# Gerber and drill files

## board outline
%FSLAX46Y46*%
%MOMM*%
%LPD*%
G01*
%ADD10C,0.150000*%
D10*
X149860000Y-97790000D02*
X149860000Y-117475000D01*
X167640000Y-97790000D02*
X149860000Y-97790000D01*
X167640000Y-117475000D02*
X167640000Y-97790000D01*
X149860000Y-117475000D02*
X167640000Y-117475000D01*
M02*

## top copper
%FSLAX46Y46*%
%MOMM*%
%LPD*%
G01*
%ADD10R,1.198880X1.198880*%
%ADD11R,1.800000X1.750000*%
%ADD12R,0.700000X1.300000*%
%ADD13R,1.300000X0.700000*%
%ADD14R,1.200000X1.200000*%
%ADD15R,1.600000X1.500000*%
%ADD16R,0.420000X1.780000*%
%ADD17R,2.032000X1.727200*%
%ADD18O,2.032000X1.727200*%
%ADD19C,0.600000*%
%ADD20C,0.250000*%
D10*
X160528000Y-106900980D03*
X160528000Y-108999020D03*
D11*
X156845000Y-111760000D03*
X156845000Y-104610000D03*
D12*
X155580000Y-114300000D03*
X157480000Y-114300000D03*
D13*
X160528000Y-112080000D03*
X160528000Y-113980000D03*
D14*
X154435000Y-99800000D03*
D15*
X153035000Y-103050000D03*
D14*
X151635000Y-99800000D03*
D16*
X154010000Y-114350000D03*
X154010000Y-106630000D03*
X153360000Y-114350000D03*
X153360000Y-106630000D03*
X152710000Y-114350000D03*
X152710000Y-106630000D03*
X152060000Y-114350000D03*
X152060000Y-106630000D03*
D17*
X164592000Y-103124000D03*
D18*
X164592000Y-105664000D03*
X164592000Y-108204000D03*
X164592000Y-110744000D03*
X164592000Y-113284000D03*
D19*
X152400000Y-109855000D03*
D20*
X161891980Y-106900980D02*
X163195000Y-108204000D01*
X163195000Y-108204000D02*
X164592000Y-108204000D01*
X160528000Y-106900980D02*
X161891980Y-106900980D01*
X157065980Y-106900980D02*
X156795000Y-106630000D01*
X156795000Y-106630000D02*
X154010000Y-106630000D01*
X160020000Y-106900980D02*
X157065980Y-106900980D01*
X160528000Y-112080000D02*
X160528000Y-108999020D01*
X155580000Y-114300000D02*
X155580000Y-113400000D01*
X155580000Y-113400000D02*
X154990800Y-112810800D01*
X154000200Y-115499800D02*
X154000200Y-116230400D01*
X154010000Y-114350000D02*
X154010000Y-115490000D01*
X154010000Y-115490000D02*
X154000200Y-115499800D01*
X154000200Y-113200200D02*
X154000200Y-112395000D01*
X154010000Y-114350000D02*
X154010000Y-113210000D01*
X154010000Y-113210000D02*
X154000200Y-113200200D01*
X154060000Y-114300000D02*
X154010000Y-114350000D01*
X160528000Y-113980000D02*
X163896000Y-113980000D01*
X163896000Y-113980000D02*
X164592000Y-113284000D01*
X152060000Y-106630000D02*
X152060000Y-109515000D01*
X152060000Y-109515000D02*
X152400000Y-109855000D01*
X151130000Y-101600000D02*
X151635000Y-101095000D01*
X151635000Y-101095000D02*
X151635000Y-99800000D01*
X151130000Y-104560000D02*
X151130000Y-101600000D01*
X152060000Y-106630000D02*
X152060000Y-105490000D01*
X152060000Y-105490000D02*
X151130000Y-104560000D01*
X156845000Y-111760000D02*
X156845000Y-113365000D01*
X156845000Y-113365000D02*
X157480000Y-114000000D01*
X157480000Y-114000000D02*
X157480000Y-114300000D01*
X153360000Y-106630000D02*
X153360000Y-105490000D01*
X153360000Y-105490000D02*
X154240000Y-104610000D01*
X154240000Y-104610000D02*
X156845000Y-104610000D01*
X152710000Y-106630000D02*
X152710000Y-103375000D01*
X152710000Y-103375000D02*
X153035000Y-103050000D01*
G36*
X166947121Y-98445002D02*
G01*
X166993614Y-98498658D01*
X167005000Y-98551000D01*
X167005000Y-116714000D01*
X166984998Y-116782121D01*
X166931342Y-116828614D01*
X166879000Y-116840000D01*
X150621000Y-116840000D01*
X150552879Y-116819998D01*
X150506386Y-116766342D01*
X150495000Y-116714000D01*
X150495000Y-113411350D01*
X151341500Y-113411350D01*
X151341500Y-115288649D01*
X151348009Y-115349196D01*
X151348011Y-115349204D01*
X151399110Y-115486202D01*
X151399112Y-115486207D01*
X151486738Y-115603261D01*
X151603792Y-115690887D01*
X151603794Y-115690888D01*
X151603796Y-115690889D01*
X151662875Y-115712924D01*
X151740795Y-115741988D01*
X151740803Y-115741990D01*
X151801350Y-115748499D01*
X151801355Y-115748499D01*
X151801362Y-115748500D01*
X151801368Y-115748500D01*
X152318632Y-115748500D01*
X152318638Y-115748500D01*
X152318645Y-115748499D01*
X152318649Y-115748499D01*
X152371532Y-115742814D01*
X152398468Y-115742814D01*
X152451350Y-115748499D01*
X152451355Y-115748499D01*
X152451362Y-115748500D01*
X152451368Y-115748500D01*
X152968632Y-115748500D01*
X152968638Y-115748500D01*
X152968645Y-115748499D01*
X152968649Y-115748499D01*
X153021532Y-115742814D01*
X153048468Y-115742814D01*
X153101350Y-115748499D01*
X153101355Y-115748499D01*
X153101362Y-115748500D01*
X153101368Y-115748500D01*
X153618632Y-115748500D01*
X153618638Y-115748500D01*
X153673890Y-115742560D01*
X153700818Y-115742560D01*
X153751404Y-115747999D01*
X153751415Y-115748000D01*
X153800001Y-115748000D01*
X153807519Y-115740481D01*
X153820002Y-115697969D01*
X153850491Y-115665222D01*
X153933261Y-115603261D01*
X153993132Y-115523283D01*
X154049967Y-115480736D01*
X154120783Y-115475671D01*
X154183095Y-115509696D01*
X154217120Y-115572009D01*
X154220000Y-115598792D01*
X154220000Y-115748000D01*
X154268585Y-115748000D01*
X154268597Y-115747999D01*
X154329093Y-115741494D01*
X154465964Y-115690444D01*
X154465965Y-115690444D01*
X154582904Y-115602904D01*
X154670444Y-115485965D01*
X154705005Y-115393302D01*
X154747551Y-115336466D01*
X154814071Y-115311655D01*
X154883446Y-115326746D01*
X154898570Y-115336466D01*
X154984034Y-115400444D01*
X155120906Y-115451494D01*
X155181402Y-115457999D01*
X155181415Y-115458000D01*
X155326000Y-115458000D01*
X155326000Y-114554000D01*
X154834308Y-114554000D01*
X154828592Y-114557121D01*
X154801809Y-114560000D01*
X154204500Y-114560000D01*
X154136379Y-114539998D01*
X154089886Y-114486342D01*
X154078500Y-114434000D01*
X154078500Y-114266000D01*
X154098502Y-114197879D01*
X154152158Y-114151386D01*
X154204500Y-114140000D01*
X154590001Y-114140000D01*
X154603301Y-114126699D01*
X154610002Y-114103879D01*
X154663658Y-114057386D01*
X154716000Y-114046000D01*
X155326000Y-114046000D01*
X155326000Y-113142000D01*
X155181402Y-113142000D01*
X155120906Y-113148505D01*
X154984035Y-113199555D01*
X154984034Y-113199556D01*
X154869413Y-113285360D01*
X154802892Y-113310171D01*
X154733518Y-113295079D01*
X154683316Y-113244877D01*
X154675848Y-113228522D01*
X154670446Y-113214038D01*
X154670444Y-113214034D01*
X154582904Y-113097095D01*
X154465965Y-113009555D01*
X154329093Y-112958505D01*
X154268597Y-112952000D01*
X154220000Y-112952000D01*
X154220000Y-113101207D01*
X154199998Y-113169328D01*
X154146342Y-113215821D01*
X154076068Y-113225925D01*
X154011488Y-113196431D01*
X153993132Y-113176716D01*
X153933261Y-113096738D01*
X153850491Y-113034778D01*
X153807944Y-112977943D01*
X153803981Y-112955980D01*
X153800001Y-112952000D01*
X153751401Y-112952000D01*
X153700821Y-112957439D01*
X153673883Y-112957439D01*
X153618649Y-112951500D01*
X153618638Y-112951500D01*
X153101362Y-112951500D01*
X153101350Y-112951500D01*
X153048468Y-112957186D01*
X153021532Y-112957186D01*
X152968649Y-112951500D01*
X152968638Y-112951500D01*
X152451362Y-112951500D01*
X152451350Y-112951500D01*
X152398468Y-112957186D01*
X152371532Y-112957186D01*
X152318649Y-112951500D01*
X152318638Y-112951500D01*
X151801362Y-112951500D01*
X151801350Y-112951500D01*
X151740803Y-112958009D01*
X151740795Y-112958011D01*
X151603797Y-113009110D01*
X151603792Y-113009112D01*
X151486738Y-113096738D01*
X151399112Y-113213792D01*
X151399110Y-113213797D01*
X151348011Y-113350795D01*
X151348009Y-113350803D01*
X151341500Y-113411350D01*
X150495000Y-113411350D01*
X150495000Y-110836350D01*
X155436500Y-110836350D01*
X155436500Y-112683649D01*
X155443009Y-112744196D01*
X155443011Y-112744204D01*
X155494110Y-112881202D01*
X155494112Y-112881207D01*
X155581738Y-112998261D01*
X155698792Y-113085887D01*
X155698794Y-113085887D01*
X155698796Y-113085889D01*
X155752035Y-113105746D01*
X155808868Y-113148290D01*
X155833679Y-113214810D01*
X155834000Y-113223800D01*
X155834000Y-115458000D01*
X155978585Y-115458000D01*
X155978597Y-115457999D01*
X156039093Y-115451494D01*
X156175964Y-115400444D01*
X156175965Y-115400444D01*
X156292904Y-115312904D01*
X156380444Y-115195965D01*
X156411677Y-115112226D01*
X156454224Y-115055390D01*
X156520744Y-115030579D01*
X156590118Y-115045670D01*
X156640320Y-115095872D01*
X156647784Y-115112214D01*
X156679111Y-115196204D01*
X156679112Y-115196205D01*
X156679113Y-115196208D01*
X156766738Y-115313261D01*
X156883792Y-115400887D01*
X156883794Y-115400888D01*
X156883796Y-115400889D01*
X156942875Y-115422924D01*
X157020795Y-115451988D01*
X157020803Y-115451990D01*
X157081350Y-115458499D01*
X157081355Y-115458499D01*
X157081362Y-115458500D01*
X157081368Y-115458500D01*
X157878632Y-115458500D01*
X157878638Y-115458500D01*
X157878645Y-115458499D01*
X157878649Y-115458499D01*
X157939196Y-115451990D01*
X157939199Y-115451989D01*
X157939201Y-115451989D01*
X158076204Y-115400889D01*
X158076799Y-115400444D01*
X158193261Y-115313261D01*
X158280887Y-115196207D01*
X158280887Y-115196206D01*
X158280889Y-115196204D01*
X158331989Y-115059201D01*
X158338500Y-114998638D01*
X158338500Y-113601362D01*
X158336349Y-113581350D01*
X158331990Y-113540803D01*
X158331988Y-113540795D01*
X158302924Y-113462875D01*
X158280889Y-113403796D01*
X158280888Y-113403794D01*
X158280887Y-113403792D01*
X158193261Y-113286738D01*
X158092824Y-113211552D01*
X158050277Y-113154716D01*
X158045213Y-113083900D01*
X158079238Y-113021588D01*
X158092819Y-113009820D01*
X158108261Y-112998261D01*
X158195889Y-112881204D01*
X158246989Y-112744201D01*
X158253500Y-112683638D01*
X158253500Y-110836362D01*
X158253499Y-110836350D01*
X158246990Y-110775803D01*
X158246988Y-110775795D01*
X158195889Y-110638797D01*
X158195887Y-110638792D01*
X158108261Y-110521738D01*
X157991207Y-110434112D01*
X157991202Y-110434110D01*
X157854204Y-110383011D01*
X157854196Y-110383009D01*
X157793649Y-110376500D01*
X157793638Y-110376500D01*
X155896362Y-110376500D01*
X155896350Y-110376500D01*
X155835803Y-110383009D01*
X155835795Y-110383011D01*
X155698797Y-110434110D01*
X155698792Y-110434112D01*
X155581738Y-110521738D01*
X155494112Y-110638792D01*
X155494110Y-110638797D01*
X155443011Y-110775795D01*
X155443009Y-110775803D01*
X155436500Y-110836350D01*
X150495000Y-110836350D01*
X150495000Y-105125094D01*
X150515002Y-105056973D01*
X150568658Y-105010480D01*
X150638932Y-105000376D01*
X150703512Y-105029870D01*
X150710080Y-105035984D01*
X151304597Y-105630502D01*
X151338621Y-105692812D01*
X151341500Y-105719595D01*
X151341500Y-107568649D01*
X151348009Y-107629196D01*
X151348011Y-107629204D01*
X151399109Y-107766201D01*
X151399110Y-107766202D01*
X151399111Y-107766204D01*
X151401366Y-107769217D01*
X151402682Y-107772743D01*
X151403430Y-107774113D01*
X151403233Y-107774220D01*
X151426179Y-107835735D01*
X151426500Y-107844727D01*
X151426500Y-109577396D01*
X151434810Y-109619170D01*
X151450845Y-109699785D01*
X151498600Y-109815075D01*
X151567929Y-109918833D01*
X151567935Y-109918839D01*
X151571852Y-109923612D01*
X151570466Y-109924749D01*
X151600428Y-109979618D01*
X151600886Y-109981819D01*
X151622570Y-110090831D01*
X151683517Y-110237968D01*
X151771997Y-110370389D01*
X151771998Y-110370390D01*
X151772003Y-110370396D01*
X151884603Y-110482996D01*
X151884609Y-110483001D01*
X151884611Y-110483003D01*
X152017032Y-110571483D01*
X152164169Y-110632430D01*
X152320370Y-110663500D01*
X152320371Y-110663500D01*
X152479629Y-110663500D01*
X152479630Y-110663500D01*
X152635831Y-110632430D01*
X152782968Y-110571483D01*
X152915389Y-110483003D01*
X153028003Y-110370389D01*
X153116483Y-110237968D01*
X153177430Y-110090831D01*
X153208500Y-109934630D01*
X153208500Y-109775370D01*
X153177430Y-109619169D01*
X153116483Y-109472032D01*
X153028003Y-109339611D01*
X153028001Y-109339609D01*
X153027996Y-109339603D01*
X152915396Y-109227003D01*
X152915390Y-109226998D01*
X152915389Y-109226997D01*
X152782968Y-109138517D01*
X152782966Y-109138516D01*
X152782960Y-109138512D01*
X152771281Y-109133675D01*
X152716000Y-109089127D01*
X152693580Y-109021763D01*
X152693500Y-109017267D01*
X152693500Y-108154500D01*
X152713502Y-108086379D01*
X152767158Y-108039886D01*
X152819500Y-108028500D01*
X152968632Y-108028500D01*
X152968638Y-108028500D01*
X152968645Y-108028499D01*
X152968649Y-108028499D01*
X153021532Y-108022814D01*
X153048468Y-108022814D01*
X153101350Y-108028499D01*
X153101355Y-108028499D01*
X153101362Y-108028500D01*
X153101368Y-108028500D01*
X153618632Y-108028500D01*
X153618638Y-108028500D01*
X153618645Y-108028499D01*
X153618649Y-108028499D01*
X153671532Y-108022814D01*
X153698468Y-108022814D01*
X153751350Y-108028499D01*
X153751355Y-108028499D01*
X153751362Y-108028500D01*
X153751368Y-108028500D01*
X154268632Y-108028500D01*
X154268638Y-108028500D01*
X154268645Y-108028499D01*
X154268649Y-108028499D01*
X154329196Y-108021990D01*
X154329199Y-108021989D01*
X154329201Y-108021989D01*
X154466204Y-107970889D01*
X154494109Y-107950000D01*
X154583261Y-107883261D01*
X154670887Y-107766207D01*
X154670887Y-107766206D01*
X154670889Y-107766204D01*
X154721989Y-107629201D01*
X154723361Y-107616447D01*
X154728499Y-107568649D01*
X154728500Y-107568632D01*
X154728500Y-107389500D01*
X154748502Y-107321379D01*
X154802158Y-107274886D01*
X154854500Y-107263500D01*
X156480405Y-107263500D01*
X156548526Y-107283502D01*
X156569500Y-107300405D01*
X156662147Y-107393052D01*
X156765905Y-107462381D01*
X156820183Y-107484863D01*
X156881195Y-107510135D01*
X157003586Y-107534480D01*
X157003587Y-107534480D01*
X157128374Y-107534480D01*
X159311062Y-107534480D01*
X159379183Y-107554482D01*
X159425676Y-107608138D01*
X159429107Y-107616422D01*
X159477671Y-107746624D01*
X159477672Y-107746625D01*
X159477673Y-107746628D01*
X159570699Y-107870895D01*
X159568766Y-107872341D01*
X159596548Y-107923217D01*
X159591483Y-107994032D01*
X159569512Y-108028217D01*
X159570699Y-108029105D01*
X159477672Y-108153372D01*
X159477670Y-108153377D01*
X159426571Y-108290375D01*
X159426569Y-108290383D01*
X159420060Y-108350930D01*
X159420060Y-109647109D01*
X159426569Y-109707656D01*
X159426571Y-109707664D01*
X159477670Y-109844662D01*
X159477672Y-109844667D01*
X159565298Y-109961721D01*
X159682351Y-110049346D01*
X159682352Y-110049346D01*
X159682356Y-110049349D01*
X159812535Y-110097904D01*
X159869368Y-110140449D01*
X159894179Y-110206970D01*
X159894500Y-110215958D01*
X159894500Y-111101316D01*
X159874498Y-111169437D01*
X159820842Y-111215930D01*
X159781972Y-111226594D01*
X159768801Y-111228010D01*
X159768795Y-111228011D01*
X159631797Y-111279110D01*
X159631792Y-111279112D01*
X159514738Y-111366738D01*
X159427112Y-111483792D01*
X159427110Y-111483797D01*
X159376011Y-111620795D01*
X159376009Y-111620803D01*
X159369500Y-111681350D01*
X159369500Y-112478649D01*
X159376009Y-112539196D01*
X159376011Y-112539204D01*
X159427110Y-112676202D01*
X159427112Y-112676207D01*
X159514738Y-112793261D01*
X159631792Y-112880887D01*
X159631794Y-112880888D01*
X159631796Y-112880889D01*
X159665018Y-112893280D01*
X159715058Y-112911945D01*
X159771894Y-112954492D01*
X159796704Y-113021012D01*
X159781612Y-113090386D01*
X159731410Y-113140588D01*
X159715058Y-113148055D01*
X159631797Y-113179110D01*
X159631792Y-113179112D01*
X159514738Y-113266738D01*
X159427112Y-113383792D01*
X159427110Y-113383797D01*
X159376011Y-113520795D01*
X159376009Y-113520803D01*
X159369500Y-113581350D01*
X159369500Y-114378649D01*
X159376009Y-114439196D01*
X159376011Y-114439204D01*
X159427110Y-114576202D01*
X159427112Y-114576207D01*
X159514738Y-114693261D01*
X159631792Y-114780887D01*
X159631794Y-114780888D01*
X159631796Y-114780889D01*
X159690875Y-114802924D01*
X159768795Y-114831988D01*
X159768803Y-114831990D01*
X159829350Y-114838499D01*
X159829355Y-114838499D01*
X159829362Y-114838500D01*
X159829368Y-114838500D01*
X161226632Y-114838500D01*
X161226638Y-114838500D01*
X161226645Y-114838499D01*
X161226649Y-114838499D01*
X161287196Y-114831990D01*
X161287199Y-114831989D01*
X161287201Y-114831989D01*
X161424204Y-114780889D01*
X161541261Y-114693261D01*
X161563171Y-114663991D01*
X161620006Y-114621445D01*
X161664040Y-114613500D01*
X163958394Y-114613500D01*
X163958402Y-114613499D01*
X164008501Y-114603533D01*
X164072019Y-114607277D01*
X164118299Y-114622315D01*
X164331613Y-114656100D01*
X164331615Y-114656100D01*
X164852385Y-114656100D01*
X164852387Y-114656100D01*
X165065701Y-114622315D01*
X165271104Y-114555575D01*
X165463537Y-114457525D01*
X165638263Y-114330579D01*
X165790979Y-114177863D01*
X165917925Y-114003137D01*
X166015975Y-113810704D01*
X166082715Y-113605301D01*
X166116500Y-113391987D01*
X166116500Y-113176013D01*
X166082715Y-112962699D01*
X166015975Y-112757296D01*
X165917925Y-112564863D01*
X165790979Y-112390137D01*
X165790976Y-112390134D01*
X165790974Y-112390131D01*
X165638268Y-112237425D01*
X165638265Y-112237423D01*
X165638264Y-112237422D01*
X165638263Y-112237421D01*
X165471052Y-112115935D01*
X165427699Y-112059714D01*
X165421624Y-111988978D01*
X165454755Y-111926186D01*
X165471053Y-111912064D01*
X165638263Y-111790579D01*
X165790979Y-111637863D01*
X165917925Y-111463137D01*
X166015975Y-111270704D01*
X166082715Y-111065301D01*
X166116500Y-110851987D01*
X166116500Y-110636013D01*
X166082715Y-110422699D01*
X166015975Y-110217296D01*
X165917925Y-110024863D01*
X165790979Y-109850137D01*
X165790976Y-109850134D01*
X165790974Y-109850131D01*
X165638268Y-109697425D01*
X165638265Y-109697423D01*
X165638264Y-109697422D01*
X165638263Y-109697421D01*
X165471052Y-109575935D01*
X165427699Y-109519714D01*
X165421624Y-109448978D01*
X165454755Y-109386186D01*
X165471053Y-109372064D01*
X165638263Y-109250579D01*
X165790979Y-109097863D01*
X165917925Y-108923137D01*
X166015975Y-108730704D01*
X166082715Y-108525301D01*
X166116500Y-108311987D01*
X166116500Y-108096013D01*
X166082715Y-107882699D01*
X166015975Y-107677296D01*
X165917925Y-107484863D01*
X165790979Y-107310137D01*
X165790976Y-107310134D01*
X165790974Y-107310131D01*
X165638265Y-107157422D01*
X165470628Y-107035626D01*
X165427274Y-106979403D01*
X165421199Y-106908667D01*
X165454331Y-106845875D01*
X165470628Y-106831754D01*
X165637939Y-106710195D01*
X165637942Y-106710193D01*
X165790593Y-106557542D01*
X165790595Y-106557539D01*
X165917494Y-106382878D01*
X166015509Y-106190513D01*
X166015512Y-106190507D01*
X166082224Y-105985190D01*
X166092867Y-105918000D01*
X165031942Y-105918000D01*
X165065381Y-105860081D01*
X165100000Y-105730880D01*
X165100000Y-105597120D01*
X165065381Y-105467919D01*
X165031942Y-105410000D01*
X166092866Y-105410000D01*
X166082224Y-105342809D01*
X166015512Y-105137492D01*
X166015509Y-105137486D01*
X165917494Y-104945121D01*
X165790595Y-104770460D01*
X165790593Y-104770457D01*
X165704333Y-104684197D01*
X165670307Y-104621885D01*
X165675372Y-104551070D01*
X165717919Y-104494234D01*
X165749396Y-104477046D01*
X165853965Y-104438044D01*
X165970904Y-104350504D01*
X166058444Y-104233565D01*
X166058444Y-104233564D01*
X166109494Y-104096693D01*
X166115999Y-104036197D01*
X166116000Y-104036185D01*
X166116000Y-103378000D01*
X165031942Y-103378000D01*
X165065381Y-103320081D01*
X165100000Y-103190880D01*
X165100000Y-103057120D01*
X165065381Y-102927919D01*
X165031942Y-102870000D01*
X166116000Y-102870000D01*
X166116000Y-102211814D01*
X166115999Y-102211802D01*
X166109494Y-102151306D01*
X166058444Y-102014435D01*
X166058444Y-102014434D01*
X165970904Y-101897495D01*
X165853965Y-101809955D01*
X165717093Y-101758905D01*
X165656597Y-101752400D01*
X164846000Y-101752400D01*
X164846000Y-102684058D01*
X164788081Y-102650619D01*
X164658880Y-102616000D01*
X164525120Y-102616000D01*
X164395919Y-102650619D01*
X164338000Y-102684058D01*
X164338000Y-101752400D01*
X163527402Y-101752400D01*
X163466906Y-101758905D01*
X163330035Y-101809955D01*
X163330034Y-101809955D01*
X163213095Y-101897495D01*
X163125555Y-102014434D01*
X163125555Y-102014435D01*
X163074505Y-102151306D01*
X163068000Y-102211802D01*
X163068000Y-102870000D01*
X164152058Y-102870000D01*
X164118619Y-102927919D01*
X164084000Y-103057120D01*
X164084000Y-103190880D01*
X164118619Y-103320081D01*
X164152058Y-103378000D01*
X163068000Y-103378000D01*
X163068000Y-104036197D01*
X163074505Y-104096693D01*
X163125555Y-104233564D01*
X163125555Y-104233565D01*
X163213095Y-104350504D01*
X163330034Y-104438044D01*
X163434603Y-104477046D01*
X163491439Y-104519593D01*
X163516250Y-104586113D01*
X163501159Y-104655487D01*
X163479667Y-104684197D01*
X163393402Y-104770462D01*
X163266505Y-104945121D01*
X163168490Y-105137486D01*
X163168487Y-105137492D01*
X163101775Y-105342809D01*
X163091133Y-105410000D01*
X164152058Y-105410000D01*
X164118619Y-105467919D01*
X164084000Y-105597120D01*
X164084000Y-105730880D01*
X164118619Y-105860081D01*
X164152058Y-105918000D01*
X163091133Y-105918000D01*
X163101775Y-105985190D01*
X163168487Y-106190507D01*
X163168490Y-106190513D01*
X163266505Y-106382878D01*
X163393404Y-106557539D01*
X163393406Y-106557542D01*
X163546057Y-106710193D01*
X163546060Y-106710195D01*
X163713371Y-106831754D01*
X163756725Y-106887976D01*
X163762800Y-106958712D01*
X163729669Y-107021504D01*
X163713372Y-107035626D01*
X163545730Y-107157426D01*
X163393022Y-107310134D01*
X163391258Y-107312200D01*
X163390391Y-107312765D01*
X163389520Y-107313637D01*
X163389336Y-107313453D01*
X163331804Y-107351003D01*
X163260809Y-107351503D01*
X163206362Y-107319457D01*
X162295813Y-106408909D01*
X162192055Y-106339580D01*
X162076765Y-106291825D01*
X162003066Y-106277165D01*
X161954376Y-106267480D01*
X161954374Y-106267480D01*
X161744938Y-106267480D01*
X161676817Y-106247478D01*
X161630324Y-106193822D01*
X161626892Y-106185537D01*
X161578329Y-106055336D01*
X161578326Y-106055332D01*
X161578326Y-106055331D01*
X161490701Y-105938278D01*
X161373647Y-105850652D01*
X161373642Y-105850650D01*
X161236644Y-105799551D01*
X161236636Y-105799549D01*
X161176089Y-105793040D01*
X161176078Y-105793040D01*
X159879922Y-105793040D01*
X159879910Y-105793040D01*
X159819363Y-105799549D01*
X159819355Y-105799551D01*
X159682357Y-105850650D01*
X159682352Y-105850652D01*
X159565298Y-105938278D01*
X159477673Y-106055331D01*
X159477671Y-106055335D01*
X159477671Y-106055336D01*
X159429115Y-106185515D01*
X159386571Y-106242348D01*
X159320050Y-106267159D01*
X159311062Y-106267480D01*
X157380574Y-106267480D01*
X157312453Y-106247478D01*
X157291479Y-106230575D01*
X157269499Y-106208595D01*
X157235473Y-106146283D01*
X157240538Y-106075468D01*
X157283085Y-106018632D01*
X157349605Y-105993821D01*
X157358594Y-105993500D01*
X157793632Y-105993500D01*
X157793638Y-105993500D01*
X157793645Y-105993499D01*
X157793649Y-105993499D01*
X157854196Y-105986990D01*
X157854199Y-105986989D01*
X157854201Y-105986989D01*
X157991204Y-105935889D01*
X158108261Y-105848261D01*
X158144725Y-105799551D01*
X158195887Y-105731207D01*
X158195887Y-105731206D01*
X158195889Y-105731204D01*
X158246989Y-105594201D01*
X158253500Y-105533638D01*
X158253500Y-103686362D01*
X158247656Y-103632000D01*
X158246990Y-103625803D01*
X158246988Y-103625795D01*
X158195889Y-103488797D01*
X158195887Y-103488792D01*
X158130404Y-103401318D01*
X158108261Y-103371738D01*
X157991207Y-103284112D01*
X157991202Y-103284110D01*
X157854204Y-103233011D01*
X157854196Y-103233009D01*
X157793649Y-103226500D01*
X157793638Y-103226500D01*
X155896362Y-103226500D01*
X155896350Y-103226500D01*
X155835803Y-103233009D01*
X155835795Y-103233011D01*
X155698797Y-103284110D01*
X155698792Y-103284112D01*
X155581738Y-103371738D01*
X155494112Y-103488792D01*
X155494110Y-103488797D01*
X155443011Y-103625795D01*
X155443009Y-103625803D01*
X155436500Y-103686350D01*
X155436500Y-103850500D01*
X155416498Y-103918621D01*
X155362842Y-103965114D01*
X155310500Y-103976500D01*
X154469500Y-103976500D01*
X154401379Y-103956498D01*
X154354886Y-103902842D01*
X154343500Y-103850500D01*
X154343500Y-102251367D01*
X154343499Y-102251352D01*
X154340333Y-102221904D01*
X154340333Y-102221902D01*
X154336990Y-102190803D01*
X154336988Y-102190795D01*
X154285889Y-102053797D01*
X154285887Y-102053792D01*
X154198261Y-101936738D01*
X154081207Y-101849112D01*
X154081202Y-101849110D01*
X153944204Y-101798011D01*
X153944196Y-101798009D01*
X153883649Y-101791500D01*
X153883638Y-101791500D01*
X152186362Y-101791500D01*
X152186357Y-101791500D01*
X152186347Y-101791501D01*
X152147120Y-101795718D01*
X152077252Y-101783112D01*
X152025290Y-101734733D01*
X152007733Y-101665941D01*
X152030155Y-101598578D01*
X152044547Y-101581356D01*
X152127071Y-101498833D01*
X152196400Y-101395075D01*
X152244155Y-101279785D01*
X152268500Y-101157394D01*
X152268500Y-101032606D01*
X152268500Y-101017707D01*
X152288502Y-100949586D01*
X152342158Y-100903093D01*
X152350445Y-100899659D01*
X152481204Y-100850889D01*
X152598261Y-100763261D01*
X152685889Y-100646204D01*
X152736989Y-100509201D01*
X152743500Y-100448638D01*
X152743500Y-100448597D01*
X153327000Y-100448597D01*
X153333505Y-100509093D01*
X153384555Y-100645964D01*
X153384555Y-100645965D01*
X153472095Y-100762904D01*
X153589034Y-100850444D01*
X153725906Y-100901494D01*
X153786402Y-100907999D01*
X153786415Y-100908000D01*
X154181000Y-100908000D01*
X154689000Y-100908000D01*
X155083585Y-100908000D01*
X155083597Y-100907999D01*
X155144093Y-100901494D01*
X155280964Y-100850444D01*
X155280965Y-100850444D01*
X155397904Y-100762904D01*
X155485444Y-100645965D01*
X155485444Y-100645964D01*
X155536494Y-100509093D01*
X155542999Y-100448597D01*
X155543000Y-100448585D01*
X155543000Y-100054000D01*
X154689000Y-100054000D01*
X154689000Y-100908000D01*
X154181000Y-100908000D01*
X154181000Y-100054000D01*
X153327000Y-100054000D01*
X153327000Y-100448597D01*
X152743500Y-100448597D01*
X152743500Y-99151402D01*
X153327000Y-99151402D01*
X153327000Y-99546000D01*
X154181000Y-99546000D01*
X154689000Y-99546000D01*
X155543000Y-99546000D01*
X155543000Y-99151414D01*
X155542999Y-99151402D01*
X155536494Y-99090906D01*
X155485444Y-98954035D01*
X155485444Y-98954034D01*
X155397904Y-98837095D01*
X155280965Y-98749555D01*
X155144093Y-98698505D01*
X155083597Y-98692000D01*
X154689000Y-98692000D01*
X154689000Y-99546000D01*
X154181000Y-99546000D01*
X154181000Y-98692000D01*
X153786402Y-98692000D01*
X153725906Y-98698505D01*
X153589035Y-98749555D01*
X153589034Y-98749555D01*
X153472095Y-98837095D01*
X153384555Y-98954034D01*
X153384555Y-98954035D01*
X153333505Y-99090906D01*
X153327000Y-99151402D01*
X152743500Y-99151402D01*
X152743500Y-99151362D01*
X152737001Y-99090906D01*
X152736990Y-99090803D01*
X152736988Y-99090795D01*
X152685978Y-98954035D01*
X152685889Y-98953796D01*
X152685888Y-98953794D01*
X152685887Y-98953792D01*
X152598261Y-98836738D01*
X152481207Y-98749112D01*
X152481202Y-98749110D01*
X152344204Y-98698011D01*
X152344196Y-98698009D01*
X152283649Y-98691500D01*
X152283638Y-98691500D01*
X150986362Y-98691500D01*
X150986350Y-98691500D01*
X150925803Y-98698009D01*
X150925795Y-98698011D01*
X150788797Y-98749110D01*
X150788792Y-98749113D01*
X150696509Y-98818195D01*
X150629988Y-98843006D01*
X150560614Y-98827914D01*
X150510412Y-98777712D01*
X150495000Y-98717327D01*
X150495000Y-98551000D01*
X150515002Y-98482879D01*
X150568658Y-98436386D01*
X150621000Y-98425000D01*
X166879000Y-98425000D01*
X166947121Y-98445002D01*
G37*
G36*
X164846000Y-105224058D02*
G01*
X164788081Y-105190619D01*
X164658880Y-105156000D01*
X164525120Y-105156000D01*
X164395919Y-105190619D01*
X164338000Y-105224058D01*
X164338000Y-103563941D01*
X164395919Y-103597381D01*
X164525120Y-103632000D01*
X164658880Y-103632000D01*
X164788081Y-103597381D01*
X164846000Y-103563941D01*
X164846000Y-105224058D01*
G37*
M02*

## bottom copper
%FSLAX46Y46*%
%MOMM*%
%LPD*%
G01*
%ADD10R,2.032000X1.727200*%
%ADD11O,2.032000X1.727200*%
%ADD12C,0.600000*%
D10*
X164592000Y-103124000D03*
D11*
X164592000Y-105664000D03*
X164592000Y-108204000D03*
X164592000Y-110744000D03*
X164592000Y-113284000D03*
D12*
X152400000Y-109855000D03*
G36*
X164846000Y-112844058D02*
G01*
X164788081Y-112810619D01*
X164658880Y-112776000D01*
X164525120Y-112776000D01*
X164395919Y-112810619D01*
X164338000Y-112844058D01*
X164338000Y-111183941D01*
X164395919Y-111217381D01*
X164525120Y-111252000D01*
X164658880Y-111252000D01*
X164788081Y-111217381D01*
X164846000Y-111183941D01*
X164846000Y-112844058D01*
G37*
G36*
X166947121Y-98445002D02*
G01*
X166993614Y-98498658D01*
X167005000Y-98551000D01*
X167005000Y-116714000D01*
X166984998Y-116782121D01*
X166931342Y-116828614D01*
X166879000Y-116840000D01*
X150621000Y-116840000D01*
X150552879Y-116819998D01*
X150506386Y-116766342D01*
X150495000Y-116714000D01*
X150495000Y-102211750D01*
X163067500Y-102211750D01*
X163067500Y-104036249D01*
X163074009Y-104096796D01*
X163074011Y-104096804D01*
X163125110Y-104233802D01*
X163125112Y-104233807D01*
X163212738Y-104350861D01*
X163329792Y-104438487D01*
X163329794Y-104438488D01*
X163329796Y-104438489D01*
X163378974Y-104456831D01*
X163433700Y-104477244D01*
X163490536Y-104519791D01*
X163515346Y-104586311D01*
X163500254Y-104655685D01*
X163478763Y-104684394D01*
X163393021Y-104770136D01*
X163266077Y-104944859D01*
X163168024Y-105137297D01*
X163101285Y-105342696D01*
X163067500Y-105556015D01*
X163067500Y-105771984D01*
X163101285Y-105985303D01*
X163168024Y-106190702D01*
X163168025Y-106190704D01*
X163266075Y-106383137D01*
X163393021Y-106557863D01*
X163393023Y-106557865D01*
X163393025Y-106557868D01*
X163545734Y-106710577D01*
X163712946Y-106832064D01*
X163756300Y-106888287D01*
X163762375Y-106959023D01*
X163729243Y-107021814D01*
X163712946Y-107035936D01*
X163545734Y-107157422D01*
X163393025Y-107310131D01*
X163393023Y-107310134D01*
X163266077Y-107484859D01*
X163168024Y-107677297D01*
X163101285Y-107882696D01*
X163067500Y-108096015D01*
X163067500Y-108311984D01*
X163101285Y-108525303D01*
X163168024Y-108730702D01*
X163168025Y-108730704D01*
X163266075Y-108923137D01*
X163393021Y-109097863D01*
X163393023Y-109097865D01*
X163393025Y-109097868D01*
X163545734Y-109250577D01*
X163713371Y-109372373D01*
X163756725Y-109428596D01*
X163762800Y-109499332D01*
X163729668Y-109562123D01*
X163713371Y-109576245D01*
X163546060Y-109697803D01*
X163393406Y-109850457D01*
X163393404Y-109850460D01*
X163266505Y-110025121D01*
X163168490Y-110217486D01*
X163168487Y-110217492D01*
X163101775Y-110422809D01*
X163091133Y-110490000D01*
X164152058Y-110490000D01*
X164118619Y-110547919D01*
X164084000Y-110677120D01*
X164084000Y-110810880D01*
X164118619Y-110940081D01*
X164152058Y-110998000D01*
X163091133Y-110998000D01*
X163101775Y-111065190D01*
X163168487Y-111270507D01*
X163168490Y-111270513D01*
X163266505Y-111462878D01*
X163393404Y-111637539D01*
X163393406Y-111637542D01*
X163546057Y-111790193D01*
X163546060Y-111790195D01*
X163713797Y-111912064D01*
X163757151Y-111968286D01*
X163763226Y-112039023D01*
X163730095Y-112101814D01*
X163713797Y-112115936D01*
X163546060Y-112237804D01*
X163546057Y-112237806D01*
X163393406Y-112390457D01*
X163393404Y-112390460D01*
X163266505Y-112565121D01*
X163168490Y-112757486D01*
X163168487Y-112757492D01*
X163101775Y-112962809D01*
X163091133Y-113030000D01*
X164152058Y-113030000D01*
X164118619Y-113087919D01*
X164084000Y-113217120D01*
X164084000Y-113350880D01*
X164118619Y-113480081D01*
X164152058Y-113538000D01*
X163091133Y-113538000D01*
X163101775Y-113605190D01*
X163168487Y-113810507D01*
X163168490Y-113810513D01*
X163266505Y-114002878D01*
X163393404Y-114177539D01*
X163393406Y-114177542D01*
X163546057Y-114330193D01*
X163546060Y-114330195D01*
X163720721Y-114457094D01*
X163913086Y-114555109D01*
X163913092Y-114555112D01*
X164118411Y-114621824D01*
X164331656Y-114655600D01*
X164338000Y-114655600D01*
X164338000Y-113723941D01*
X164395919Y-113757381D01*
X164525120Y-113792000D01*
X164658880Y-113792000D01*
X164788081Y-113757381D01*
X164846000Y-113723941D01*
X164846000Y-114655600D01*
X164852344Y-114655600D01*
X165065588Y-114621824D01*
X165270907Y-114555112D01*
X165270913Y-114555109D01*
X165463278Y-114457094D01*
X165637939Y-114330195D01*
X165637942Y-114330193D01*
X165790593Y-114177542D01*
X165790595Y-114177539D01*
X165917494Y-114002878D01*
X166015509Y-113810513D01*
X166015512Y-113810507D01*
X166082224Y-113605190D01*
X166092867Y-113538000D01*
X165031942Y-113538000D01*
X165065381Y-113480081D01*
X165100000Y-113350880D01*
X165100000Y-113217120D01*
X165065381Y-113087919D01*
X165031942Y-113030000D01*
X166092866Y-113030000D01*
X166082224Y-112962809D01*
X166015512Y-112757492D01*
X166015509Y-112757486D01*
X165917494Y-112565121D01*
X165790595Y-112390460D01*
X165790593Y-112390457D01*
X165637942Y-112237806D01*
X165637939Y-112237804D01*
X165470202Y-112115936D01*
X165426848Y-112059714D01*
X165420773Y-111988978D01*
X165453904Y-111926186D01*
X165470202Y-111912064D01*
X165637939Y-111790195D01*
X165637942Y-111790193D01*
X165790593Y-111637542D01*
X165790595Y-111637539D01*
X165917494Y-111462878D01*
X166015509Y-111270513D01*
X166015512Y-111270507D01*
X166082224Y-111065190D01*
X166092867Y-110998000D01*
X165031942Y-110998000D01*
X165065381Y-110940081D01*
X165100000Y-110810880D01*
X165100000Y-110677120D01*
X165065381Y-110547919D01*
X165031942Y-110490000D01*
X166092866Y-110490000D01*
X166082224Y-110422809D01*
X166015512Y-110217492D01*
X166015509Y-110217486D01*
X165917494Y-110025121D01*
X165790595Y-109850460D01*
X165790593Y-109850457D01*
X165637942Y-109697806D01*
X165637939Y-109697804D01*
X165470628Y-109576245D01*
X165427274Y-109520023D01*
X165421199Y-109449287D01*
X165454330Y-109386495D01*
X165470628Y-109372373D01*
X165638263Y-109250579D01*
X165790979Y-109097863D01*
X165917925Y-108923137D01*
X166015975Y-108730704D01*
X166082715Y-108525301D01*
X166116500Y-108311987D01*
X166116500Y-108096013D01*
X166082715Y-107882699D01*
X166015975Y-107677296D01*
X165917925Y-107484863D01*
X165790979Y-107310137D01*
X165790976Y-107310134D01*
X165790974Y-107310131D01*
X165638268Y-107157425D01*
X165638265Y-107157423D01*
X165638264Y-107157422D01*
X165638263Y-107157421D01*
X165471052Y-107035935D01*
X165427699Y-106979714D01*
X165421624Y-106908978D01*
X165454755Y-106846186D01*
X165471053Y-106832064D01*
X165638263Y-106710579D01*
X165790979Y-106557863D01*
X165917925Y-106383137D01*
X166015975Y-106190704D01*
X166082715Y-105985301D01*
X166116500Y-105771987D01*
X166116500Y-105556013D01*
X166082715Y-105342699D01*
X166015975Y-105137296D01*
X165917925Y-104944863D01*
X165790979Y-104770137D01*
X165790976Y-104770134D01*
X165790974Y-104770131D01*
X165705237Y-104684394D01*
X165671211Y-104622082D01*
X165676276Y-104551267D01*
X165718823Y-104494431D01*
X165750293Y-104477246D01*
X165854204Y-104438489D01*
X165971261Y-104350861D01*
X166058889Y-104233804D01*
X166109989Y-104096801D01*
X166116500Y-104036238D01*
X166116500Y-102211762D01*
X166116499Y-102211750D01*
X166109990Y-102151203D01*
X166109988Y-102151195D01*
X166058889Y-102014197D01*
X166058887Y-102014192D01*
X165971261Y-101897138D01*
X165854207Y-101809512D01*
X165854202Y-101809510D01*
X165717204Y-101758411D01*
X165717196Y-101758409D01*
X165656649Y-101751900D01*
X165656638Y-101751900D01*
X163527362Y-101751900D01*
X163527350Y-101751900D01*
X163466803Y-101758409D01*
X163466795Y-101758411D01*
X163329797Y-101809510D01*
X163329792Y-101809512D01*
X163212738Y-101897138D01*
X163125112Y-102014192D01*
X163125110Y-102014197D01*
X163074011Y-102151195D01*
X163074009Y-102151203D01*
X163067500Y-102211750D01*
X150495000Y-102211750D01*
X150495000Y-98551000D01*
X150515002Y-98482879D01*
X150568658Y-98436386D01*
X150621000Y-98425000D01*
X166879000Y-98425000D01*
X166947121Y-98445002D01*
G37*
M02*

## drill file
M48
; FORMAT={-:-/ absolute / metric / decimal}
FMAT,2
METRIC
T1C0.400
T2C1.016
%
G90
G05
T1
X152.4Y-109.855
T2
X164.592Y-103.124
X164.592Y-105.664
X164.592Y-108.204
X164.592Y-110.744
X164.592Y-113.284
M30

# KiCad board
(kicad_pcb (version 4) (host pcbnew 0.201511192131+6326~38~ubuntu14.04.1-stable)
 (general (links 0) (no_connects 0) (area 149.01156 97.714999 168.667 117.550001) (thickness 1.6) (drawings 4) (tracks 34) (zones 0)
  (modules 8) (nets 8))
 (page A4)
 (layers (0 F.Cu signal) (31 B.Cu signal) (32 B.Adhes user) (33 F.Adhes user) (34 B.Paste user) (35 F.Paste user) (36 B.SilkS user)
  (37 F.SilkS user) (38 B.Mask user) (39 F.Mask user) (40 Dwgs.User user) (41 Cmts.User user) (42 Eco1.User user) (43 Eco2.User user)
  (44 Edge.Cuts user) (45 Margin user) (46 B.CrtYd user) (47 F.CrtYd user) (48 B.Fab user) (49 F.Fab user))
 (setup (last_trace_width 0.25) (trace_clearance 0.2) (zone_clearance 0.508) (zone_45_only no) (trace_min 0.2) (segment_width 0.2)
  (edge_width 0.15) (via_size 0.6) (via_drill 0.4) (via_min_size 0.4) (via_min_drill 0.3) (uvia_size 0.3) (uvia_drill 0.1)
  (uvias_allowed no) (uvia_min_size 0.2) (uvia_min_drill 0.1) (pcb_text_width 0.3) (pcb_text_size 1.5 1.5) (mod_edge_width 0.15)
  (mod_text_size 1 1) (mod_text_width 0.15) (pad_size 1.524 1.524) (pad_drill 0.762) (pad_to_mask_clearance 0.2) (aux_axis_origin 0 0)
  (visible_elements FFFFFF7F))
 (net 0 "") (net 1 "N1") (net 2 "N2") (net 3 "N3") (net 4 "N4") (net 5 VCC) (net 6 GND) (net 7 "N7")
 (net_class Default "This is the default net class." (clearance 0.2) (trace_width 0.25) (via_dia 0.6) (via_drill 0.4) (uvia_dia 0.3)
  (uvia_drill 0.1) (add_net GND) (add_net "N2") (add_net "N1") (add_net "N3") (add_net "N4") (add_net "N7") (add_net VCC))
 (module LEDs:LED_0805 (layer F.Cu) (at 160.528 107.95 90)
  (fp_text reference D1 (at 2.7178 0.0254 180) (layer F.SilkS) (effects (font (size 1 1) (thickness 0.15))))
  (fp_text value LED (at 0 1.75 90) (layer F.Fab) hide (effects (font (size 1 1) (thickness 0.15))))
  (pad 2 smd rect (at 1.04902 0 270) (size 1.19888 1.19888) (layers F.Cu F.Paste F.Mask) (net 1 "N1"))
  (pad 1 smd rect (at -1.04902 0 270) (size 1.19888 1.19888) (layers F.Cu F.Paste F.Mask) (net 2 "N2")))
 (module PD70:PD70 (layer F.Cu) (at 156.845 108.185 90)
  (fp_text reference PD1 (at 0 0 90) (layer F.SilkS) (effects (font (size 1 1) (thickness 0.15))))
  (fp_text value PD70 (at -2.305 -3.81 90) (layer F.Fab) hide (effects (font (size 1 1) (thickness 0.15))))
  (pad 1 smd rect (at -3.575 0 90) (size 1.75 1.8) (layers F.Cu F.Paste F.Mask) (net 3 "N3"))
  (pad 2 smd rect (at 3.575 0 90) (size 1.75 1.8) (layers F.Cu F.Paste F.Mask) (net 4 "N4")))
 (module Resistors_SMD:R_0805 (layer F.Cu) (at 156.53 114.3)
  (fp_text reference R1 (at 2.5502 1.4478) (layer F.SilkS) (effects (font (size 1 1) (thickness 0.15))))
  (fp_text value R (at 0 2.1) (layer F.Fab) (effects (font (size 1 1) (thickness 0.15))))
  (pad 1 smd rect (at -0.95 0) (size 0.7 1.3) (layers F.Cu F.Paste F.Mask) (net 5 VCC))
  (pad 2 smd rect (at 0.95 0) (size 0.7 1.3) (layers F.Cu F.Paste F.Mask) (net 3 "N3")))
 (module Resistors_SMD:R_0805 (layer F.Cu) (at 160.528 113.03 270)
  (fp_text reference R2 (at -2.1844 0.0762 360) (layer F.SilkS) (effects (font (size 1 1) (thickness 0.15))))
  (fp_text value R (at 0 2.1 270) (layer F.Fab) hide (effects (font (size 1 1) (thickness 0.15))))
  (pad 1 smd rect (at -0.95 0 270) (size 0.7 1.3) (layers F.Cu F.Paste F.Mask) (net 2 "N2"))
  (pad 2 smd rect (at 0.95 0 270) (size 0.7 1.3) (layers F.Cu F.Paste F.Mask) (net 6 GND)))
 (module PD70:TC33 (layer F.Cu) (at 153.035 101.6 180)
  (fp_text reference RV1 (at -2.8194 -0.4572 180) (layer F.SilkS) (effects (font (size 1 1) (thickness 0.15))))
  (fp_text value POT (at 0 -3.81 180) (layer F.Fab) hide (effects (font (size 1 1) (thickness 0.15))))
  (pad 1 smd rect (at -1.4 1.8 180) (size 1.2 1.2) (layers F.Cu F.Paste F.Mask) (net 5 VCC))
  (pad 2 smd rect (at 0 -1.45 180) (size 1.6 1.5) (layers F.Cu F.Paste F.Mask) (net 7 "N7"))
  (pad 3 smd rect (at 1.4 1.8 180) (size 1.2 1.2) (layers F.Cu F.Paste F.Mask) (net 6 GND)))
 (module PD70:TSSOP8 (layer F.Cu) (at 153.035 110.49 180)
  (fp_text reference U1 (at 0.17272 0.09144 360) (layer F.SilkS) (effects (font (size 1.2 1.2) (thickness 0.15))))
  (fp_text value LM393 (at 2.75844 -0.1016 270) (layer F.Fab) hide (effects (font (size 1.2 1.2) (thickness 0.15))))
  (pad 8 smd rect (at -0.975 -3.86 180) (size 0.42 1.78) (layers F.Cu F.Paste F.Mask) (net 5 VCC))
  (pad 1 smd rect (at -0.975 3.86 180) (size 0.42 1.78) (layers F.Cu F.Paste F.Mask) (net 1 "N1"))
  (pad 7 smd rect (at -0.325 -3.86 180) (size 0.42 1.78) (layers F.Cu F.Paste F.Mask))
  (pad 2 smd rect (at -0.325 3.86 180) (size 0.42 1.78) (layers F.Cu F.Paste F.Mask) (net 4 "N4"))
  (pad 6 smd rect (at 0.325 -3.86 180) (size 0.42 1.78) (layers F.Cu F.Paste F.Mask))
  (pad 3 smd rect (at 0.325 3.86 180) (size 0.42 1.78) (layers F.Cu F.Paste F.Mask) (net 7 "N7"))
  (pad 5 smd rect (at 0.975 -3.86 180) (size 0.42 1.78) (layers F.Cu F.Paste F.Mask))
  (pad 4 smd rect (at 0.975 3.86 180) (size 0.42 1.78) (layers F.Cu F.Paste F.Mask) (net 6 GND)))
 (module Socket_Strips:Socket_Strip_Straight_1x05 (layer F.Cu) (at 164.592 103.124 270)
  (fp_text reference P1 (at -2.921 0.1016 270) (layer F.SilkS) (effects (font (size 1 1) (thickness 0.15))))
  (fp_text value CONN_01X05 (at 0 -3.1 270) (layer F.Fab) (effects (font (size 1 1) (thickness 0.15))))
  (pad 1 thru_hole rect (at 0 0 270) (size 1.7272 2.032) (drill 1.016) (layers *.Cu *.Mask F.SilkS) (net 5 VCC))
  (pad 2 thru_hole oval (at 2.54 0 270) (size 1.7272 2.032) (drill 1.016) (layers *.Cu *.Mask F.SilkS) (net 5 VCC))
  (pad 3 thru_hole oval (at 5.08 0 270) (size 1.7272 2.032) (drill 1.016) (layers *.Cu *.Mask F.SilkS) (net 1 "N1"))
  (pad 4 thru_hole oval (at 7.62 0 270) (size 1.7272 2.032) (drill 1.016) (layers *.Cu *.Mask F.SilkS) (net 6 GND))
  (pad 5 thru_hole oval (at 10.16 0 270) (size 1.7272 2.032) (drill 1.016) (layers *.Cu *.Mask F.SilkS) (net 6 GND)))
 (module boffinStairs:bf (layer F.Cu) (at 159.9946 100.7364)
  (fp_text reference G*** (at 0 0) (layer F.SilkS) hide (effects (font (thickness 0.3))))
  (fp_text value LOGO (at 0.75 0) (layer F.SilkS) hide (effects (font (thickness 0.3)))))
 (gr_line (start 149.86 97.79) (end 149.86 117.475) (layer Edge.Cuts) (width 0.15))
 (gr_line (start 167.64 97.79) (end 149.86 97.79) (layer Edge.Cuts) (width 0.15))
 (gr_line (start 167.64 117.475) (end 167.64 97.79) (layer Edge.Cuts) (width 0.15))
 (gr_line (start 149.86 117.475) (end 167.64 117.475) (layer Edge.Cuts) (width 0.15))
 (segment (start 161.89198 106.90098) (end 163.195 108.204) (width 0.25) (layer F.Cu) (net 1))
 (segment (start 163.195 108.204) (end 164.592 108.204) (width 0.25) (layer F.Cu) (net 1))
 (segment (start 160.528 106.90098) (end 161.89198 106.90098) (width 0.25) (layer F.Cu) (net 1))
 (segment (start 157.06598 106.90098) (end 156.795 106.63) (width 0.25) (layer F.Cu) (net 1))
 (segment (start 156.795 106.63) (end 154.01 106.63) (width 0.25) (layer F.Cu) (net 1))
 (segment (start 160.02 106.90098) (end 157.06598 106.90098) (width 0.25) (layer F.Cu) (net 1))
 (segment (start 160.528 112.08) (end 160.528 108.99902) (width 0.25) (layer F.Cu) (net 2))
 (segment (start 155.58 114.3) (end 155.58 113.4) (width 0.25) (layer F.Cu) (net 5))
 (segment (start 155.58 113.4) (end 154.9908 112.8108) (width 0.25) (layer F.Cu) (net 5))
 (segment (start 154.0002 115.4998) (end 154.0002 116.2304) (width 0.25) (layer F.Cu) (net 5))
 (segment (start 154.01 114.35) (end 154.01 115.49) (width 0.25) (layer F.Cu) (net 5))
 (segment (start 154.01 115.49) (end 154.0002 115.4998) (width 0.25) (layer F.Cu) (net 5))
 (segment (start 154.0002 113.2002) (end 154.0002 112.395) (width 0.25) (layer F.Cu) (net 5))
 (segment (start 154.01 114.35) (end 154.01 113.21) (width 0.25) (layer F.Cu) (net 5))
 (segment (start 154.01 113.21) (end 154.0002 113.2002) (width 0.25) (layer F.Cu) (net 5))
 (segment (start 154.06 114.3) (end 154.01 114.35) (width 0.25) (layer F.Cu) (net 5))
 (segment (start 160.528 113.98) (end 163.896 113.98) (width 0.25) (layer F.Cu) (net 6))
 (segment (start 163.896 113.98) (end 164.592 113.284) (width 0.25) (layer F.Cu) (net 6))
 (segment (start 152.06 106.63) (end 152.06 109.515) (width 0.25) (layer F.Cu) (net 6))
 (segment (start 152.06 109.515) (end 152.4 109.855) (width 0.25) (layer F.Cu) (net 6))
 (via (at 152.4 109.855) (size 0.6) (drill 0.4) (layers F.Cu B.Cu) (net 6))
 (segment (start 151.13 101.6) (end 151.635 101.095) (width 0.25) (layer F.Cu) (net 6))
 (segment (start 151.635 101.095) (end 151.635 99.8) (width 0.25) (layer F.Cu) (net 6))
 (segment (start 151.13 104.56) (end 151.13 101.6) (width 0.25) (layer F.Cu) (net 6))
 (segment (start 152.06 106.63) (end 152.06 105.49) (width 0.25) (layer F.Cu) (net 6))
 (segment (start 152.06 105.49) (end 151.13 104.56) (width 0.25) (layer F.Cu) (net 6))
 (segment (start 156.845 111.76) (end 156.845 113.365) (width 0.25) (layer F.Cu) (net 3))
 (segment (start 156.845 113.365) (end 157.48 114) (width 0.25) (layer F.Cu) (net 3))
 (segment (start 157.48 114) (end 157.48 114.3) (width 0.25) (layer F.Cu) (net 3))
 (segment (start 153.36 106.63) (end 153.36 105.49) (width 0.25) (layer F.Cu) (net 4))
 (segment (start 153.36 105.49) (end 154.24 104.61) (width 0.25) (layer F.Cu) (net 4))
 (segment (start 154.24 104.61) (end 156.845 104.61) (width 0.25) (layer F.Cu) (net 4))
 (segment (start 152.71 106.63) (end 152.71 103.375) (width 0.25) (layer F.Cu) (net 7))
 (segment (start 152.71 103.375) (end 153.035 103.05) (width 0.25) (layer F.Cu) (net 7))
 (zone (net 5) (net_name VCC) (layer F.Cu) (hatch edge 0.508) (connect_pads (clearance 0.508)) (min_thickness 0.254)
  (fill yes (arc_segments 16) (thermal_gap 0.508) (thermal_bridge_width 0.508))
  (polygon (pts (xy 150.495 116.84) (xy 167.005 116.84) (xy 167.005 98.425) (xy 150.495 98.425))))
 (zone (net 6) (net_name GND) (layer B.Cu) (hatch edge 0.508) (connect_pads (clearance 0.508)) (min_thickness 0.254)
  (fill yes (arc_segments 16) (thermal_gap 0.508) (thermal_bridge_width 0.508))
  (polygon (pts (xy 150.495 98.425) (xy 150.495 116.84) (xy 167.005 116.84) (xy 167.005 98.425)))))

